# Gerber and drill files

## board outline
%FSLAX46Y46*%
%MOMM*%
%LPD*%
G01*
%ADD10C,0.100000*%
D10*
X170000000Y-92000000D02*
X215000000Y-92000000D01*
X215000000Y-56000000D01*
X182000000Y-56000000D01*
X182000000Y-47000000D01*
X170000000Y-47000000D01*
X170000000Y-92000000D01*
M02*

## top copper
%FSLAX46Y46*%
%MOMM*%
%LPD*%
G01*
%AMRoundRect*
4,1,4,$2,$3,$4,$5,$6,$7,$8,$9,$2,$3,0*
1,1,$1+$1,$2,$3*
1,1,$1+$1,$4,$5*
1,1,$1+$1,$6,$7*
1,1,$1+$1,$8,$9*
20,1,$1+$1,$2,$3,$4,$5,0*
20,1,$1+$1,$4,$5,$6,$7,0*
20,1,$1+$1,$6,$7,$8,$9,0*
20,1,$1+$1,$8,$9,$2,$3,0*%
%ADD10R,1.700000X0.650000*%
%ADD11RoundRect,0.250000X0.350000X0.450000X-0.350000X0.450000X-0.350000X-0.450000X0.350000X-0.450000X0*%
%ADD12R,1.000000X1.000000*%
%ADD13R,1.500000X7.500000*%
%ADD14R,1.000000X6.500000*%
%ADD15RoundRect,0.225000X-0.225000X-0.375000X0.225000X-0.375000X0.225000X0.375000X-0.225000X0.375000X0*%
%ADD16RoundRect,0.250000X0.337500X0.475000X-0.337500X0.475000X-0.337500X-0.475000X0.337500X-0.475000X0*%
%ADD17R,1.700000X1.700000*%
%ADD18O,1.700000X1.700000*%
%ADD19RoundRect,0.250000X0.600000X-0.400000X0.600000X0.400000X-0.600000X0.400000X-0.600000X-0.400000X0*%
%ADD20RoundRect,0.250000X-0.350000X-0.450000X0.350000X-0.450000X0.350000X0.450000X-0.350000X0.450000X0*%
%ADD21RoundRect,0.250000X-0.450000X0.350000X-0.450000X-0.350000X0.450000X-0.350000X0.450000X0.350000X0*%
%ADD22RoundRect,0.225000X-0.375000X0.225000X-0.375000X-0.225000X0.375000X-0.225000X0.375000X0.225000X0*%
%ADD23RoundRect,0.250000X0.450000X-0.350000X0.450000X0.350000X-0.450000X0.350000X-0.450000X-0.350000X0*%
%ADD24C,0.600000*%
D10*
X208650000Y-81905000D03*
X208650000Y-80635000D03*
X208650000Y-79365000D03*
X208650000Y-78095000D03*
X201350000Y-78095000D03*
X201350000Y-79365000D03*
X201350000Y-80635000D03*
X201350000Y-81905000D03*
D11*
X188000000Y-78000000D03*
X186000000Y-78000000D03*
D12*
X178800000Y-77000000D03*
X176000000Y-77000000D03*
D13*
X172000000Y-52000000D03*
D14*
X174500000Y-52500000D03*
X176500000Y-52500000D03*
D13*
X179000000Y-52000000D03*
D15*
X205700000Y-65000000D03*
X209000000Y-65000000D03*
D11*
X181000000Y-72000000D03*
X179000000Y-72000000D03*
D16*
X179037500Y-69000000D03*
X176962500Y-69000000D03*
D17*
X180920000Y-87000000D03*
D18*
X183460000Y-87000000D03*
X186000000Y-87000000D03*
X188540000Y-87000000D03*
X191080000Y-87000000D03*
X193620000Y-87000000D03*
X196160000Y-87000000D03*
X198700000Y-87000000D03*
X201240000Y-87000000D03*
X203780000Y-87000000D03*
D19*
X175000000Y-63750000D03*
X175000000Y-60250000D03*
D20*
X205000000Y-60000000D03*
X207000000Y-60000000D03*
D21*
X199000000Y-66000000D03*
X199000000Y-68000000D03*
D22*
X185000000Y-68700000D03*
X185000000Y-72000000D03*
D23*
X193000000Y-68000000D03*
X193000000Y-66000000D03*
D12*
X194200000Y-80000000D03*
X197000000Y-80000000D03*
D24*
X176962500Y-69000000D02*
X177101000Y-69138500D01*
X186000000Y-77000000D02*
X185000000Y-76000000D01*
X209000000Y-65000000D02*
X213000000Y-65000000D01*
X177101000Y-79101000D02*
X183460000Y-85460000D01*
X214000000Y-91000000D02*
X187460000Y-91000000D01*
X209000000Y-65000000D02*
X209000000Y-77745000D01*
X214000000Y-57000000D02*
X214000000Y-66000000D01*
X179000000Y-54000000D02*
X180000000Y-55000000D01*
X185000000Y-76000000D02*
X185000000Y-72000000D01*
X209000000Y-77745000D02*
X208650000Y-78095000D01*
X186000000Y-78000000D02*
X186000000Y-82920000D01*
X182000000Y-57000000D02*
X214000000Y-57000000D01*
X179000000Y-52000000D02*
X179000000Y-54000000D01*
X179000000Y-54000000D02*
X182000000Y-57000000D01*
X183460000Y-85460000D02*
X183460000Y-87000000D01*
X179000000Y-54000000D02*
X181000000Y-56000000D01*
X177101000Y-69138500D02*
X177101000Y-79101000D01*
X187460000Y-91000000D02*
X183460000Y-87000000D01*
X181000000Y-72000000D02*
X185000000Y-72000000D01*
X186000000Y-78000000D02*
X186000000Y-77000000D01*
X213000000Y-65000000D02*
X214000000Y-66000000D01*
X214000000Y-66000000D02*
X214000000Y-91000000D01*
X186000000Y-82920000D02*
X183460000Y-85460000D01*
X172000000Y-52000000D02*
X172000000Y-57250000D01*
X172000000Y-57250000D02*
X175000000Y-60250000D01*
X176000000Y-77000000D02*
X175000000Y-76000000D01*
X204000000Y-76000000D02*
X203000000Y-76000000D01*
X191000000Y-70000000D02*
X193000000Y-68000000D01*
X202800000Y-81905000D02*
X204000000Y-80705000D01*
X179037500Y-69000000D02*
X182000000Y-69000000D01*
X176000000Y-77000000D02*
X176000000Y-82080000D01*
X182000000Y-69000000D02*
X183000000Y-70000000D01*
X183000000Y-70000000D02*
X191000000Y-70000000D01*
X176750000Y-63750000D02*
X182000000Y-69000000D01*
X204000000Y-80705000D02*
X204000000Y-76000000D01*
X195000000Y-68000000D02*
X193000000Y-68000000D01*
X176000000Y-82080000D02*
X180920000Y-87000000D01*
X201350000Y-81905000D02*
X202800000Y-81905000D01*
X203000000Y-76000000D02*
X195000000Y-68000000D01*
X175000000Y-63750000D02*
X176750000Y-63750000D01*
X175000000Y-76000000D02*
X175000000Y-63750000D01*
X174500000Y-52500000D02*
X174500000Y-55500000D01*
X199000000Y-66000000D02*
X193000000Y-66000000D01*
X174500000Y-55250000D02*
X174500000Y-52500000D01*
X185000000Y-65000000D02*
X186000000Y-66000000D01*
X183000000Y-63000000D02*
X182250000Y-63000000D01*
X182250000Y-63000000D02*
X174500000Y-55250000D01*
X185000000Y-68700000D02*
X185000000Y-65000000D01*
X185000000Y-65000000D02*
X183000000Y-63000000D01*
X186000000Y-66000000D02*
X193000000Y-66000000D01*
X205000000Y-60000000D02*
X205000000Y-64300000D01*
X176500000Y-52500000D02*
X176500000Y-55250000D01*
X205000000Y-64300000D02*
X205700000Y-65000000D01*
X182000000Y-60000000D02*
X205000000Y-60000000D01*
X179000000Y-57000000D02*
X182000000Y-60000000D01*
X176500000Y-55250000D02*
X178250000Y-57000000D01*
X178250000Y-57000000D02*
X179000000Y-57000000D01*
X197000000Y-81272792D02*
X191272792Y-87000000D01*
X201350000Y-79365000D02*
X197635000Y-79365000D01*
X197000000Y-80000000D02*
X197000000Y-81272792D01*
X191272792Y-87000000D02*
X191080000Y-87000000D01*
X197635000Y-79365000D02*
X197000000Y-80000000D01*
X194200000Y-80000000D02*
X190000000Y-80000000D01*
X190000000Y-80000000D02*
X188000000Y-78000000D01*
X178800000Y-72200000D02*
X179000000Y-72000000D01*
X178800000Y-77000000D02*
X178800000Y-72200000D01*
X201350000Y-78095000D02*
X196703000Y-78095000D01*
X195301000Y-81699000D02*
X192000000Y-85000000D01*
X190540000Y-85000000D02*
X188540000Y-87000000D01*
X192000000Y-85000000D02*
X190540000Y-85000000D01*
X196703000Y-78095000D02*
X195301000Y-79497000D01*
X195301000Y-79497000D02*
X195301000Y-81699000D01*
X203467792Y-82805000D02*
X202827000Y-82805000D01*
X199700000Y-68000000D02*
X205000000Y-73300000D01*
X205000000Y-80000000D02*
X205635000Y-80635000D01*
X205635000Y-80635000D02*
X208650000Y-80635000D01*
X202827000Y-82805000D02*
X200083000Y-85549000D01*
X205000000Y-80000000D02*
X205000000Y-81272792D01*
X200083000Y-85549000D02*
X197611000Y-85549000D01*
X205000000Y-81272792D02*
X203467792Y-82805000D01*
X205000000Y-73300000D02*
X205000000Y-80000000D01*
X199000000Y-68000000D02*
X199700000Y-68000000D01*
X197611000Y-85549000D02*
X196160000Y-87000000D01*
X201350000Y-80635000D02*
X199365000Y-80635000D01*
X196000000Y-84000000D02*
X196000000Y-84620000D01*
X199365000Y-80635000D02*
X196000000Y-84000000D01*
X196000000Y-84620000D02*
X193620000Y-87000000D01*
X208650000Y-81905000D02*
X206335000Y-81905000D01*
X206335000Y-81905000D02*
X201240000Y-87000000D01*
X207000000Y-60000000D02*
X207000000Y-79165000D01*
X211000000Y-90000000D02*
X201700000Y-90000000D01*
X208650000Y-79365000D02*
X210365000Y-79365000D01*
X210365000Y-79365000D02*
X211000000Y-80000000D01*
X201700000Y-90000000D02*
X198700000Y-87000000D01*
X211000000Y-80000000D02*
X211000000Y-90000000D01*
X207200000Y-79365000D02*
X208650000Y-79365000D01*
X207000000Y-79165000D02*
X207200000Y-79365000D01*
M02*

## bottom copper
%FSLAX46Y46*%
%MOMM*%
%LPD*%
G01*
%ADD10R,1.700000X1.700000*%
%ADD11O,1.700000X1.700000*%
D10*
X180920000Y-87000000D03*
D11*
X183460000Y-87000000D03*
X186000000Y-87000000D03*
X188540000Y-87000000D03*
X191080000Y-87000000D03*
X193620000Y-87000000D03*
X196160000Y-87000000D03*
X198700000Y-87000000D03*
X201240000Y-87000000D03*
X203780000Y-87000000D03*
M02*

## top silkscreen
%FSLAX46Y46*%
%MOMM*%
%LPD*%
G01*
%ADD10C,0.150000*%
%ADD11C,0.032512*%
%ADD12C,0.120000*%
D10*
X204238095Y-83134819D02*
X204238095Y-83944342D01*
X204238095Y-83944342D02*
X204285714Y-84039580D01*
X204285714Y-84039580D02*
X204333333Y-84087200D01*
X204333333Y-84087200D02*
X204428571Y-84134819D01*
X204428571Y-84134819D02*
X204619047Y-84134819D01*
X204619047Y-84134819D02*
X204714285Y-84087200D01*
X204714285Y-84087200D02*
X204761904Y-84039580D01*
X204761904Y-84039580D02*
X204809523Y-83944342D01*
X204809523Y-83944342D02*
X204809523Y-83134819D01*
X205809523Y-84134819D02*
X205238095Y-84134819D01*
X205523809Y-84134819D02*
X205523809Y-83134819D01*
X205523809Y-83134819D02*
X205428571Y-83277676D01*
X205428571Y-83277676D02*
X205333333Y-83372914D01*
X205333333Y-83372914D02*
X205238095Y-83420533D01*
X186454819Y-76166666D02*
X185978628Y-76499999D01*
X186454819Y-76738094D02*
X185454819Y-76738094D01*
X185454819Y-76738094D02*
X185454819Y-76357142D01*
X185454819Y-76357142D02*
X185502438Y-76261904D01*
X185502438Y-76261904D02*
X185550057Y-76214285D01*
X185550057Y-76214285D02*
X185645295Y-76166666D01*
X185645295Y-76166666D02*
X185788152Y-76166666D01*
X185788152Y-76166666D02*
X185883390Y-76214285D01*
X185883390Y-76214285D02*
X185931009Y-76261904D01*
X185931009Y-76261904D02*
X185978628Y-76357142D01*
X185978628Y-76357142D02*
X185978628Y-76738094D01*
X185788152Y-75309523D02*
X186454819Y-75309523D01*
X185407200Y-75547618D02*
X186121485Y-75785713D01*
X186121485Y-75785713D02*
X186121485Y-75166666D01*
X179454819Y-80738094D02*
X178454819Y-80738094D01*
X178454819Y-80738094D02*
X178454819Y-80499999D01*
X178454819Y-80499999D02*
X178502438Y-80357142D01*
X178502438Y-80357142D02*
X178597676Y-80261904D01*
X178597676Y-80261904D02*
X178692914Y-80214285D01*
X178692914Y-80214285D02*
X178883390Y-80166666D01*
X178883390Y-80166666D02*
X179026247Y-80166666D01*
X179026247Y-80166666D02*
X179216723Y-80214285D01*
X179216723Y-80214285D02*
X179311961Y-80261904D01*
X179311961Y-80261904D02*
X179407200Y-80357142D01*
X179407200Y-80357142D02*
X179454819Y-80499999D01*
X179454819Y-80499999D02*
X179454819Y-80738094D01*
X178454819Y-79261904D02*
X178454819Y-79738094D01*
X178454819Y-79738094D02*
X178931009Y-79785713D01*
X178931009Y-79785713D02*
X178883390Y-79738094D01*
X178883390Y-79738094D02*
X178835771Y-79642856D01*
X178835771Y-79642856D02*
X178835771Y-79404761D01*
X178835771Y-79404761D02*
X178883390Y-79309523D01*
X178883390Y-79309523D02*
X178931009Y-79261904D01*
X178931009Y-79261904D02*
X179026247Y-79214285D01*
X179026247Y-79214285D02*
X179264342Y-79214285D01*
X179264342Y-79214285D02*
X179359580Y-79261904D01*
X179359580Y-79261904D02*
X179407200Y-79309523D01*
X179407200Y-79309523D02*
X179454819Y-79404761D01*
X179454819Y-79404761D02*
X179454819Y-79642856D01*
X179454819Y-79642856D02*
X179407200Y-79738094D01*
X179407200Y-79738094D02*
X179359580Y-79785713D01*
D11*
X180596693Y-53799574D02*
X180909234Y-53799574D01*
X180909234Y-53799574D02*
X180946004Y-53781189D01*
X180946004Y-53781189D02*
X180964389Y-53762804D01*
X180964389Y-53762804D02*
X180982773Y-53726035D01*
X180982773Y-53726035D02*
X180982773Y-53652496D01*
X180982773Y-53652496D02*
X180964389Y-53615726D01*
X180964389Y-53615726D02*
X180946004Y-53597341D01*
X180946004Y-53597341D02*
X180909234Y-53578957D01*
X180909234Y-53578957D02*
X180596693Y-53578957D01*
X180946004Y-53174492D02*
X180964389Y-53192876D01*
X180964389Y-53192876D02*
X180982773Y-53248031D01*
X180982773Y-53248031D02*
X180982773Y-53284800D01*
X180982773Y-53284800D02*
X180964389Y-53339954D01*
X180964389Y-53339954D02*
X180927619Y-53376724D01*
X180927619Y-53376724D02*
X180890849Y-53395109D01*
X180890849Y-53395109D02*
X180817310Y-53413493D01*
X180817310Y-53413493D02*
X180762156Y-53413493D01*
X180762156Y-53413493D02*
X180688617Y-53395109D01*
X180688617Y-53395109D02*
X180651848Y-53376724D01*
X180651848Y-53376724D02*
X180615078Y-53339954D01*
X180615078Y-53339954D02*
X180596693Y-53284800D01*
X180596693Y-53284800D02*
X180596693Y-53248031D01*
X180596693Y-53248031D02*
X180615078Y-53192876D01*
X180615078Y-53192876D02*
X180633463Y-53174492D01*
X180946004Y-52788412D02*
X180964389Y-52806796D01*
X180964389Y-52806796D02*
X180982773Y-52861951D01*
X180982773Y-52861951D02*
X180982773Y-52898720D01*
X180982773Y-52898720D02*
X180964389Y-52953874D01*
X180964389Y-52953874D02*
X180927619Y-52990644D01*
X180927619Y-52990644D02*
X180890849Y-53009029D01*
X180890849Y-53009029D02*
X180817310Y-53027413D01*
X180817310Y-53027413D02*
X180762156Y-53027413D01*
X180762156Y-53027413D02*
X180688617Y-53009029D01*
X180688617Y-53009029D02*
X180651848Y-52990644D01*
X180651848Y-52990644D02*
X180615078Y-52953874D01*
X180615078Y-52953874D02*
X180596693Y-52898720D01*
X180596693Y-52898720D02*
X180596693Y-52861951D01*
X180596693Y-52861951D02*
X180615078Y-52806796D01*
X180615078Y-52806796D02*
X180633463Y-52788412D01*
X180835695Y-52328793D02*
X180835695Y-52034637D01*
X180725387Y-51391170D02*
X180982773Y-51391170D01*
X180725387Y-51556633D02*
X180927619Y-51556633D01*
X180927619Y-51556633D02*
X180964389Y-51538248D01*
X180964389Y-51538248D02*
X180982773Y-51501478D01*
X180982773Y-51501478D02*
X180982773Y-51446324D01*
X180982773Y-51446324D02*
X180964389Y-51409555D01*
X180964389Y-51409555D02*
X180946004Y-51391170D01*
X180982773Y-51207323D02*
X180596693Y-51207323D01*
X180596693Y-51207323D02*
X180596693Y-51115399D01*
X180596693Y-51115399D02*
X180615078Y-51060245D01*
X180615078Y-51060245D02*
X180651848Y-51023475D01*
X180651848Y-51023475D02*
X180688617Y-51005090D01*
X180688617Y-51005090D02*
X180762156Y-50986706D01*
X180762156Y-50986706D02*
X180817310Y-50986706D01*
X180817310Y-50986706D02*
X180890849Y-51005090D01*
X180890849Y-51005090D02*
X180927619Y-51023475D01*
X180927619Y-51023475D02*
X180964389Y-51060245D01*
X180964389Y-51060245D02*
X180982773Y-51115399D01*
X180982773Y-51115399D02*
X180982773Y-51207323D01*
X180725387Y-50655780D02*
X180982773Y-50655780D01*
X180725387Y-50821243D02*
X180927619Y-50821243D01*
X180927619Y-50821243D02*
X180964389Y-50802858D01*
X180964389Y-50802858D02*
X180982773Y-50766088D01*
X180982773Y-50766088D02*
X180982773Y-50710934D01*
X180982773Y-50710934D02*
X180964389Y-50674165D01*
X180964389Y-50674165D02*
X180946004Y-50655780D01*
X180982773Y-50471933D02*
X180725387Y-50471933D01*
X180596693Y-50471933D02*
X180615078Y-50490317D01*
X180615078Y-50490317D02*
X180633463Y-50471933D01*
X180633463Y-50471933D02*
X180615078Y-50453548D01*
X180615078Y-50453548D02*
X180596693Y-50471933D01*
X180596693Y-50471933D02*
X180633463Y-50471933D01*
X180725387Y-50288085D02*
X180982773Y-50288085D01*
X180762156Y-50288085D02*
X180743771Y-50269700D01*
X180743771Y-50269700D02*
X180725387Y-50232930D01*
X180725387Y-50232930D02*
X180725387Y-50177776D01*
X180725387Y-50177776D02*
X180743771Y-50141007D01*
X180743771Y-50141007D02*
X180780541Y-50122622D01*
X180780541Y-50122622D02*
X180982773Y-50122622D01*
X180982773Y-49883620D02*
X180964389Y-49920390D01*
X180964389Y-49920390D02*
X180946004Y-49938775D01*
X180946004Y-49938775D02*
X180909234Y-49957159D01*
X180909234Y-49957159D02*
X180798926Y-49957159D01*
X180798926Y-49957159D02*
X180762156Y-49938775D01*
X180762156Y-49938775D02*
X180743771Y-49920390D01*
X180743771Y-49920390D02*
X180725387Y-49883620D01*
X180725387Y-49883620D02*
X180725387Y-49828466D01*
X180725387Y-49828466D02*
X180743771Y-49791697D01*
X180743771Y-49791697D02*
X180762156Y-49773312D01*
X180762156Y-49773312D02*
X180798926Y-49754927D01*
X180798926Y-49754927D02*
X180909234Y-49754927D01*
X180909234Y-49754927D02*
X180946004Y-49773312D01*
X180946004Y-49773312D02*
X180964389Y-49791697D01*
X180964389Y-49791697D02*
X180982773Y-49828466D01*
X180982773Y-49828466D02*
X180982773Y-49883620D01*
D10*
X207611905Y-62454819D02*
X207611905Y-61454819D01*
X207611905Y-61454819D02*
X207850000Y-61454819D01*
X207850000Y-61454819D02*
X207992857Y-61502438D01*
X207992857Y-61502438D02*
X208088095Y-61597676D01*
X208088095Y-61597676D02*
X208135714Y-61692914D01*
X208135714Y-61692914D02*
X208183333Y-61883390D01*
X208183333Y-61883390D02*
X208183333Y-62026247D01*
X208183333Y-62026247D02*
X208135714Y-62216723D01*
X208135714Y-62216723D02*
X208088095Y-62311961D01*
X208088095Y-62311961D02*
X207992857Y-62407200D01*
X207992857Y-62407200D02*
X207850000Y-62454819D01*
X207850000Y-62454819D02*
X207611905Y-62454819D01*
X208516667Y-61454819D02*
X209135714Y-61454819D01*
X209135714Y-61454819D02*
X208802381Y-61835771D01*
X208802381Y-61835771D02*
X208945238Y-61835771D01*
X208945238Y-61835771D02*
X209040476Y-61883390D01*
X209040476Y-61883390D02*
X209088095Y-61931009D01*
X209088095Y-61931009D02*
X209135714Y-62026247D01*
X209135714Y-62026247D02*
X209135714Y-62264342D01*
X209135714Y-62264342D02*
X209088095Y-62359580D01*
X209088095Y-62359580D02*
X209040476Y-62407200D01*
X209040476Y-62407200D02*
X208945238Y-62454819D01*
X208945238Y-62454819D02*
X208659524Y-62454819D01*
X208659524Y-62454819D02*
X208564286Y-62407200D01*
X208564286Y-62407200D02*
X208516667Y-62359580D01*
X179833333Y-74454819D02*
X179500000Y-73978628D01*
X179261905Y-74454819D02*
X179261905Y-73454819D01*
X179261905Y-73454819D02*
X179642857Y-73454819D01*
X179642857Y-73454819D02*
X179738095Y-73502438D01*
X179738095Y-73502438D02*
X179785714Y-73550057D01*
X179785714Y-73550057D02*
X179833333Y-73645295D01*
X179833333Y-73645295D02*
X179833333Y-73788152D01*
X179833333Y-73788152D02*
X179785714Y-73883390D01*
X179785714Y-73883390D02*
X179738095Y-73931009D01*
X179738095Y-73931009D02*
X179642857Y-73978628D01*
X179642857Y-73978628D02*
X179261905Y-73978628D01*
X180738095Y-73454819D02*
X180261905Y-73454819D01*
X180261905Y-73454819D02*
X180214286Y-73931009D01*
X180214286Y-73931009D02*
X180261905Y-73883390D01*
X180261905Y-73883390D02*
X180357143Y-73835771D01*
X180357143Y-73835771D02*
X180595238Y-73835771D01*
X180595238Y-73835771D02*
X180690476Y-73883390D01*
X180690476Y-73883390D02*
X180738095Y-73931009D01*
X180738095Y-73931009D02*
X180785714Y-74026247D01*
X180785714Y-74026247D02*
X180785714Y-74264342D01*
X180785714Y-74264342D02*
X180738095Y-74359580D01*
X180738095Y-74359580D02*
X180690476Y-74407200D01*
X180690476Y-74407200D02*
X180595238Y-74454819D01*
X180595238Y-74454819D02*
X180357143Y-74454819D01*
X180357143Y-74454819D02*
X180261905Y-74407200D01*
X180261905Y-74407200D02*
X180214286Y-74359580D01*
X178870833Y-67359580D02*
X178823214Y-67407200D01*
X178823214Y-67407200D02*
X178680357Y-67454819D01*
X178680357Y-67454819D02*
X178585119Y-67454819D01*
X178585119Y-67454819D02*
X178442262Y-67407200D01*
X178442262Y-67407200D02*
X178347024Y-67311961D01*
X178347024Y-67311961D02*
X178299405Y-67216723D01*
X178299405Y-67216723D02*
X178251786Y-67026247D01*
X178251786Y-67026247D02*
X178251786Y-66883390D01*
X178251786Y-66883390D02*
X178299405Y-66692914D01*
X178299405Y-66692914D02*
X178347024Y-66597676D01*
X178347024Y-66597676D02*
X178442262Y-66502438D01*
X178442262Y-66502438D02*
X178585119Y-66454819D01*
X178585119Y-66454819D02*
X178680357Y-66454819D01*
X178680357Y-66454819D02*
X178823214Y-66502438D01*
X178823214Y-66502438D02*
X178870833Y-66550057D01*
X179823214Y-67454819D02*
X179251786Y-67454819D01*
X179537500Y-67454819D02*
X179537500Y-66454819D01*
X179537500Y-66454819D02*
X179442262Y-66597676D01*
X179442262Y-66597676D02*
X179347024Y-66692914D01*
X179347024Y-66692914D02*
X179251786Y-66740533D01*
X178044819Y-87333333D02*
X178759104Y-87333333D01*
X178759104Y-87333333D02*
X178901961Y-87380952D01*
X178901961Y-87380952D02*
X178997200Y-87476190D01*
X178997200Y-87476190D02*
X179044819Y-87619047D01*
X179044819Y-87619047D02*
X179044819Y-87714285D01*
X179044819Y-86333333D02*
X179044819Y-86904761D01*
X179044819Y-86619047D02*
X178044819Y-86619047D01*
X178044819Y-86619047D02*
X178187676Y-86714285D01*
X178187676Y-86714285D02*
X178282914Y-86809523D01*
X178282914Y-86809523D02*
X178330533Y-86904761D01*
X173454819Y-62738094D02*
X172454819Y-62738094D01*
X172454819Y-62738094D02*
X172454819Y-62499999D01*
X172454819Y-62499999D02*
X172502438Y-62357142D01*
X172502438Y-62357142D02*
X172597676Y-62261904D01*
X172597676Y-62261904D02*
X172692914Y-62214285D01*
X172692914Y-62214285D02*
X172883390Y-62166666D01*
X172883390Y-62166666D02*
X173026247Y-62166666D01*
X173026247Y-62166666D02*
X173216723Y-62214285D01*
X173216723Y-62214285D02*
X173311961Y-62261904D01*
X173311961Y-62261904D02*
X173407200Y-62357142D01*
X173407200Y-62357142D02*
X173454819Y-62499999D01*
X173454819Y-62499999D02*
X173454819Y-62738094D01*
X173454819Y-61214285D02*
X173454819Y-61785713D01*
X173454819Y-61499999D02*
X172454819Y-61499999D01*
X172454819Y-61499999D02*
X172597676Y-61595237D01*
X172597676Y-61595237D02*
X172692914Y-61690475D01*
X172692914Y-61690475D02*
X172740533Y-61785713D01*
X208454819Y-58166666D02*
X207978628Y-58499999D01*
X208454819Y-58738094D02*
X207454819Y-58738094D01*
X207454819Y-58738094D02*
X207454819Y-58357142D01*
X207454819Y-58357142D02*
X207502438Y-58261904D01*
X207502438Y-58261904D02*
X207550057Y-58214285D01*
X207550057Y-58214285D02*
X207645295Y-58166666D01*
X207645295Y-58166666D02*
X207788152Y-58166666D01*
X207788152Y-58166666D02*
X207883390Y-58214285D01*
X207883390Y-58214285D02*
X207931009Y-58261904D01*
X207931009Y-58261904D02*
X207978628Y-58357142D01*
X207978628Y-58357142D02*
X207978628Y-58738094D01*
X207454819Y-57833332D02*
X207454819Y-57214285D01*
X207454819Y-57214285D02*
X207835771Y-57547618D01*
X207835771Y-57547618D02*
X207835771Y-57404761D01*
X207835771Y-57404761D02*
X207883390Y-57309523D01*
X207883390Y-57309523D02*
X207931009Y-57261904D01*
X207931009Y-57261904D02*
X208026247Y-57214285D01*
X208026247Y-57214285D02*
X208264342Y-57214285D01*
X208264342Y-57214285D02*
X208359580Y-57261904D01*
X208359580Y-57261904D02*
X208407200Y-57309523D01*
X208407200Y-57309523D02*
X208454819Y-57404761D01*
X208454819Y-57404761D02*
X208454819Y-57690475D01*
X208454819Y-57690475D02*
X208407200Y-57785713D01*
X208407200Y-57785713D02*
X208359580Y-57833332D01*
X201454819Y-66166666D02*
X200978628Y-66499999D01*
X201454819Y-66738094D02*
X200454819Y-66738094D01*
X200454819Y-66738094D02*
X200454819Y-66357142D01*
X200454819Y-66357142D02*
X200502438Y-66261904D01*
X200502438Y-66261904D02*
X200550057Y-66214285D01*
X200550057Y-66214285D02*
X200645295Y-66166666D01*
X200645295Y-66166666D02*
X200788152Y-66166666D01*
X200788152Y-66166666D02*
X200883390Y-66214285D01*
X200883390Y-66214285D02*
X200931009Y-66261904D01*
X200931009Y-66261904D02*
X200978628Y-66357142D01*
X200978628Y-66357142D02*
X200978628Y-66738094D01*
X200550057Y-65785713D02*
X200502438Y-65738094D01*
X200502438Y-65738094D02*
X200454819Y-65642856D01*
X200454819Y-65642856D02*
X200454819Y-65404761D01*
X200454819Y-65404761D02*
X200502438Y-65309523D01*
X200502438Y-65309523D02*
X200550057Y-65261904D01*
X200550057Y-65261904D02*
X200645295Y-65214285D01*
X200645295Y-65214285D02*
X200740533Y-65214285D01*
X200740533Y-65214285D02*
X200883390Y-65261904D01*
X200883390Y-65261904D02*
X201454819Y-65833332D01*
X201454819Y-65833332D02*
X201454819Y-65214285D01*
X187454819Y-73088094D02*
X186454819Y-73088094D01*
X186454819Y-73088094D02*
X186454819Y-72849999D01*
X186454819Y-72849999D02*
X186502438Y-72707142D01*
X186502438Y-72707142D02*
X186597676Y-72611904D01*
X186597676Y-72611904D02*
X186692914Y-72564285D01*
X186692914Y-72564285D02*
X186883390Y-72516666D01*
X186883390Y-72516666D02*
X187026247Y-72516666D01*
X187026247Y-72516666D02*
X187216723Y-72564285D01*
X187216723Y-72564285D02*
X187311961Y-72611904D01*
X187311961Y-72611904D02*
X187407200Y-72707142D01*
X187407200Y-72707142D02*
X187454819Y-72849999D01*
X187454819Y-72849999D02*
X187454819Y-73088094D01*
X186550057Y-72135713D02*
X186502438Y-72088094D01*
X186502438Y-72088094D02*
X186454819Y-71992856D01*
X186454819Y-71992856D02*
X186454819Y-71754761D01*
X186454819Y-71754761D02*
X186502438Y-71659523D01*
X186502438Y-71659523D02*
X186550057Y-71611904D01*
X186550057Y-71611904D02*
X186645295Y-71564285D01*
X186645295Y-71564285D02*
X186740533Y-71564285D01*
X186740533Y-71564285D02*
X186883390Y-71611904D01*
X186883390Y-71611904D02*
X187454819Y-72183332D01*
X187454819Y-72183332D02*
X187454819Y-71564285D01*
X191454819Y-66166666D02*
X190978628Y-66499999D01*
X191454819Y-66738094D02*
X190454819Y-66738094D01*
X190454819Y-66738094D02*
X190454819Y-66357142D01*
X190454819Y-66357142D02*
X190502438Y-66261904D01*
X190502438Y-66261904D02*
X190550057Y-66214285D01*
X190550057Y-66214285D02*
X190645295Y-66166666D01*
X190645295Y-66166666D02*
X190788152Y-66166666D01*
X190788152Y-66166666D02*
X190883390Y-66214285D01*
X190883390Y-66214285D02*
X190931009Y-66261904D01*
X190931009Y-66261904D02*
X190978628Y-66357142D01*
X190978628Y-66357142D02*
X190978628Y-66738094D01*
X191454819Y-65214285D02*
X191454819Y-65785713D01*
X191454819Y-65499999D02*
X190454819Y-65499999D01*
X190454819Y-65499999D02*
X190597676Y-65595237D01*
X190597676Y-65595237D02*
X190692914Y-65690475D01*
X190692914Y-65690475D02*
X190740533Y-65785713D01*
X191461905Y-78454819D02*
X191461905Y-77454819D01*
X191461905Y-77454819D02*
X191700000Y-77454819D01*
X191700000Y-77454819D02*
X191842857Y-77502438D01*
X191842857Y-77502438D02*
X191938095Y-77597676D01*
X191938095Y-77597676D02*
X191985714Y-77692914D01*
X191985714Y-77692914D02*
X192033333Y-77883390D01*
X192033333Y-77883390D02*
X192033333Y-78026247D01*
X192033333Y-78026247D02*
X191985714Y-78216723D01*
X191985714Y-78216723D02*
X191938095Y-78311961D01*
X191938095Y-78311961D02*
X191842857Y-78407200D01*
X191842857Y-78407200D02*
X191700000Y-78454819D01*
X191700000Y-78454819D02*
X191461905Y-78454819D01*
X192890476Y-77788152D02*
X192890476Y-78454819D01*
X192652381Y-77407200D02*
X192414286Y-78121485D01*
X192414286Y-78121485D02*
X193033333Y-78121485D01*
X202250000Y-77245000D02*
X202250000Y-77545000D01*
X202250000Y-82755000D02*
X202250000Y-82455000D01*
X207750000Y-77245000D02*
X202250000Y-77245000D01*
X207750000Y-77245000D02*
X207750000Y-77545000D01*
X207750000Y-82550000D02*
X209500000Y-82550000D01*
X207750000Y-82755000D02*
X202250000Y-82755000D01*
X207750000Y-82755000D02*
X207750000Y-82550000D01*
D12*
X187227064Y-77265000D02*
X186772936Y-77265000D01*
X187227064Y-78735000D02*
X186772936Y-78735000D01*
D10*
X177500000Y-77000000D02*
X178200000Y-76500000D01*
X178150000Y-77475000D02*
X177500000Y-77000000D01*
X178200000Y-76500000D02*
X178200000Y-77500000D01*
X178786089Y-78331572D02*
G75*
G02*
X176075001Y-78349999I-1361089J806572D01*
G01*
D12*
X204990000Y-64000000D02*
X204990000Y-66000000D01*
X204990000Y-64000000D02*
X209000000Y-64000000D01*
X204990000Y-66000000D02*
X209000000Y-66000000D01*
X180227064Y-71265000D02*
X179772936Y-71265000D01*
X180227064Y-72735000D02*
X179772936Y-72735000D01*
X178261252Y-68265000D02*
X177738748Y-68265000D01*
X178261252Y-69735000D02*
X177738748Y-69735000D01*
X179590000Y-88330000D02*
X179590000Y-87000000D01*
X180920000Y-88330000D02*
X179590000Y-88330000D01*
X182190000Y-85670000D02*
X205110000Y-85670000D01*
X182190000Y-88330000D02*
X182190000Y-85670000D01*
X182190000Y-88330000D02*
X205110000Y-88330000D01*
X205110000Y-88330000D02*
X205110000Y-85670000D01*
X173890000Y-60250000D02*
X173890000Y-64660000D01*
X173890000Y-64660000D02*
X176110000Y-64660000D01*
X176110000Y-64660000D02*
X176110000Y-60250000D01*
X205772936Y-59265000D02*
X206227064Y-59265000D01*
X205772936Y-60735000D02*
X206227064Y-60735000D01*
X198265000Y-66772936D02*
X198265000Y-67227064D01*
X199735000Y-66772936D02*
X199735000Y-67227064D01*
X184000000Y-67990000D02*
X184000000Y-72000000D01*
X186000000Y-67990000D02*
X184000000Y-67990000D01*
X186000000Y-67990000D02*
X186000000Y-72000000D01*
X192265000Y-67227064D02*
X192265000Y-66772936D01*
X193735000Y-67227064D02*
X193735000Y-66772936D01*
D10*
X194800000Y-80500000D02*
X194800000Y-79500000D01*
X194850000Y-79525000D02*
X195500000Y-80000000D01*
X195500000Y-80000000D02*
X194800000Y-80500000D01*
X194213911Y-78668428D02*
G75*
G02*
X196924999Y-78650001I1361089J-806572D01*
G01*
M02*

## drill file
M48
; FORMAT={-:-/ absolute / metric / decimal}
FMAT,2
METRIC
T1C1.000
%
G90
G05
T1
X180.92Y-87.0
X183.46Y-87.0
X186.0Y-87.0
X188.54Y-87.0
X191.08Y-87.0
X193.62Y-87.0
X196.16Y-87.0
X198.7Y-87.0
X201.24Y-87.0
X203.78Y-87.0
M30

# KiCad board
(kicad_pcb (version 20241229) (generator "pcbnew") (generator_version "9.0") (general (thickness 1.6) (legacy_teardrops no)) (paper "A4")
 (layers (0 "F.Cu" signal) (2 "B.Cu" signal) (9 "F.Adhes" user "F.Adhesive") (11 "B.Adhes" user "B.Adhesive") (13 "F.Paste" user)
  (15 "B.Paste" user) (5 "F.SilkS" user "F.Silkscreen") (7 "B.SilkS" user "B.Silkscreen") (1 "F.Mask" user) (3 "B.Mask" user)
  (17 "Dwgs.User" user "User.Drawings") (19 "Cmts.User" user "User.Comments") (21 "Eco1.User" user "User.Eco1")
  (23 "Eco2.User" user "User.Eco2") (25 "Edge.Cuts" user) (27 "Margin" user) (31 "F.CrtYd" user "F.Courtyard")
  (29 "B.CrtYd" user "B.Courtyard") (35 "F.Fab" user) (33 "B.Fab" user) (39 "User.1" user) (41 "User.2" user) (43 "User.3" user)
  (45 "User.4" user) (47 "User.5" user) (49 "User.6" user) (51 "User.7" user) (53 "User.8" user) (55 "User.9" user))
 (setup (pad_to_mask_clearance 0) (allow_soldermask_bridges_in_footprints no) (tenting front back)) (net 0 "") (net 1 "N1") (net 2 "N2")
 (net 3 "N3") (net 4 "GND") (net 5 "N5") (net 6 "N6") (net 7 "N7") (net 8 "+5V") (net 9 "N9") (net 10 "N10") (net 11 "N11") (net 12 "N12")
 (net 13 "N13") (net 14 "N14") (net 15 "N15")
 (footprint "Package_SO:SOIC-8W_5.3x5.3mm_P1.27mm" (layer "F.Cu") (at 205 80 180)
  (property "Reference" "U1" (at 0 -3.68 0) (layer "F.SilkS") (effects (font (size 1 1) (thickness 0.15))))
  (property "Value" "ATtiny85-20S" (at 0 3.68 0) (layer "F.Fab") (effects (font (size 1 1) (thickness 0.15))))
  (fp_line (start 2.75 2.755) (end 2.75 2.455) (stroke (width 0.15) (type solid)) (layer "F.SilkS"))
  (fp_line (start 2.75 -2.755) (end 2.75 -2.455) (stroke (width 0.15) (type solid)) (layer "F.SilkS"))
  (fp_line (start -2.75 2.755) (end 2.75 2.755) (stroke (width 0.15) (type solid)) (layer "F.SilkS"))
  (fp_line (start -2.75 2.755) (end -2.75 2.455) (stroke (width 0.15) (type solid)) (layer "F.SilkS"))
  (fp_line (start -2.75 -2.55) (end -4.5 -2.55) (stroke (width 0.15) (type solid)) (layer "F.SilkS"))
  (fp_line (start -2.75 -2.755) (end 2.75 -2.755) (stroke (width 0.15) (type solid)) (layer "F.SilkS"))
  (fp_line (start -2.75 -2.755) (end -2.75 -2.55) (stroke (width 0.15) (type solid)) (layer "F.SilkS"))
  (pad "1" smd rect (at -3.65 -1.905 180) (size 1.7 0.65) (layers "F.Cu" "F.Mask" "F.Paste") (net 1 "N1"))
  (pad "2" smd rect (at -3.65 -0.635 180) (size 1.7 0.65) (layers "F.Cu" "F.Mask" "F.Paste") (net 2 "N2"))
  (pad "3" smd rect (at -3.65 0.635 180) (size 1.7 0.65) (layers "F.Cu" "F.Mask" "F.Paste") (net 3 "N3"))
  (pad "4" smd rect (at -3.65 1.905 180) (size 1.7 0.65) (layers "F.Cu" "F.Mask" "F.Paste") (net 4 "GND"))
  (pad "5" smd rect (at 3.65 1.905 180) (size 1.7 0.65) (layers "F.Cu" "F.Mask" "F.Paste") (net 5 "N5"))
  (pad "6" smd rect (at 3.65 0.635 180) (size 1.7 0.65) (layers "F.Cu" "F.Mask" "F.Paste") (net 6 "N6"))
  (pad "7" smd rect (at 3.65 -0.635 180) (size 1.7 0.65) (layers "F.Cu" "F.Mask" "F.Paste") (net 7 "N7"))
  (pad "8" smd rect (at 3.65 -1.905 180) (size 1.7 0.65) (layers "F.Cu" "F.Mask" "F.Paste") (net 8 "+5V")))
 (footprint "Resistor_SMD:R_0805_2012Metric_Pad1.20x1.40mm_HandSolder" (layer "F.Cu") (at 187 78 180)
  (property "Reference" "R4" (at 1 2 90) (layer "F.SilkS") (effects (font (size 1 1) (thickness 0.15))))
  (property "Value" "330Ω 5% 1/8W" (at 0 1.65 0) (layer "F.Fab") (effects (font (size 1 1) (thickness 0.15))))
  (fp_line (start -0.227064 0.735) (end 0.227064 0.735) (stroke (width 0.12) (type solid)) (layer "F.SilkS"))
  (fp_line (start -0.227064 -0.735) (end 0.227064 -0.735) (stroke (width 0.12) (type solid)) (layer "F.SilkS"))
  (pad "1" smd roundrect (at -1 0 180) (size 1.2 1.4) (layers "F.Cu" "F.Mask" "F.Paste") (roundrect_rratio 0.208333) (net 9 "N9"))
  (pad "2" smd roundrect (at 1 0 180) (size 1.2 1.4) (layers "F.Cu" "F.Mask" "F.Paste") (roundrect_rratio 0.208333) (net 4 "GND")))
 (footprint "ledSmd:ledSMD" (layer "F.Cu") (at 177 77 180)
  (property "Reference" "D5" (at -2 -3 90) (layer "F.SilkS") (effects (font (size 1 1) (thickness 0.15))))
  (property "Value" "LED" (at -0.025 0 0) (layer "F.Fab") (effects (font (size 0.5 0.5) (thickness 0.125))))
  (fp_line (start -0.5 0) (end -1.2 0.5) (stroke (width 0.15) (type solid)) (layer "F.SilkS"))
  (fp_line (start -1.15 -0.475) (end -0.5 0) (stroke (width 0.15) (type solid)) (layer "F.SilkS"))
  (fp_line (start -1.2 0.5) (end -1.2 -0.5) (stroke (width 0.15) (type solid)) (layer "F.SilkS"))
  (fp_arc (start -1.786089 -1.331572) (mid -0.435753 -2.107089) (end 0.924999 -1.349999) (stroke (width 0.15) (type solid))
   (layer "F.SilkS"))
  (pad "1" smd rect (at -1.8 0 180) (size 1 1) (layers "F.Cu" "F.Mask" "F.Paste") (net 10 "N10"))
  (pad "2" smd rect (at 1 0 180) (size 1 1) (layers "F.Cu" "F.Mask" "F.Paste") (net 8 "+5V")))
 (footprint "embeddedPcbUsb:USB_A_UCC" (layer "F.Cu") (at 175.5 52.2 -90)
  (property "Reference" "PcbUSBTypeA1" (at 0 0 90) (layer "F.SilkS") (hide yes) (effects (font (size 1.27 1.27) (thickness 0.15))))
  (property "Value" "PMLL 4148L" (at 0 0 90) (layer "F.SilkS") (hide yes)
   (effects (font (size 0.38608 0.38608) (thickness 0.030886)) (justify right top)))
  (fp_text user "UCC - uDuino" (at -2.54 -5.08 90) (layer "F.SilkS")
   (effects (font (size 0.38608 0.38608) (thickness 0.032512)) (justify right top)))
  (pad "1" smd rect (at -0.2 3.5 270) (size 7.5 1.5) (layers "F.Cu" "F.Mask" "F.Paste") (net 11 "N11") (solder_mask_margin 0.1016))
  (pad "2" smd rect (at 0.3 1 270) (size 6.5 1) (layers "F.Cu" "F.Mask" "F.Paste") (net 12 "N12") (solder_mask_margin 0.1016))
  (pad "3" smd rect (at 0.3 -1 270) (size 6.5 1) (layers "F.Cu" "F.Mask" "F.Paste") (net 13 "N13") (solder_mask_margin 0.1016))
  (pad "4" smd rect (at -0.2 -3.5 270) (size 7.5 1.5) (layers "F.Cu" "F.Mask" "F.Paste") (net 4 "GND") (solder_mask_margin 0.1016)))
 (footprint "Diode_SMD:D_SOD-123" (layer "F.Cu") (at 207.35 65)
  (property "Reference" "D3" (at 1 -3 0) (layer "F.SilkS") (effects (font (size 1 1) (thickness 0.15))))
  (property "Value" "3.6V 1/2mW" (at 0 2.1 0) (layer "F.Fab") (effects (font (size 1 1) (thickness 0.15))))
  (fp_line (start -2.36 -1) (end -2.36 1) (stroke (width 0.12) (type solid)) (layer "F.SilkS"))
  (fp_line (start -2.36 -1) (end 1.65 -1) (stroke (width 0.12) (type solid)) (layer "F.SilkS"))
  (fp_line (start -2.36 1) (end 1.65 1) (stroke (width 0.12) (type solid)) (layer "F.SilkS"))
  (pad "1" smd roundrect (at -1.65 0) (size 0.9 1.2) (layers "F.Cu" "F.Mask" "F.Paste") (roundrect_rratio 0.25) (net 13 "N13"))
  (pad "2" smd roundrect (at 1.65 0) (size 0.9 1.2) (layers "F.Cu" "F.Mask" "F.Paste") (roundrect_rratio 0.25) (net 4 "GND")))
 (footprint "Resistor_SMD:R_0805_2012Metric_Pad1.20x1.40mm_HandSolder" (layer "F.Cu") (at 180 72 180)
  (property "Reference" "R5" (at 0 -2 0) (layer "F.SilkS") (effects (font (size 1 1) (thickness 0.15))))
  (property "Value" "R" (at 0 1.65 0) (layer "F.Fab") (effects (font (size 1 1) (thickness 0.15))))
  (fp_line (start -0.227064 0.735) (end 0.227064 0.735) (stroke (width 0.12) (type solid)) (layer "F.SilkS"))
  (fp_line (start -0.227064 -0.735) (end 0.227064 -0.735) (stroke (width 0.12) (type solid)) (layer "F.SilkS"))
  (pad "1" smd roundrect (at -1 0 180) (size 1.2 1.4) (layers "F.Cu" "F.Mask" "F.Paste") (roundrect_rratio 0.208333) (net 4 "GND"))
  (pad "2" smd roundrect (at 1 0 180) (size 1.2 1.4) (layers "F.Cu" "F.Mask" "F.Paste") (roundrect_rratio 0.208333) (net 10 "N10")))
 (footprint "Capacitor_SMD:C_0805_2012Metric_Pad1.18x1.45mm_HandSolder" (layer "F.Cu") (at 178 69 180)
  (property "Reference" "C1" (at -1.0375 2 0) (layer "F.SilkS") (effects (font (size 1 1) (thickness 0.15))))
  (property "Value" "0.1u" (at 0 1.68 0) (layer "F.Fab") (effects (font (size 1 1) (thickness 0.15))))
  (fp_line (start -0.261252 0.735) (end 0.261252 0.735) (stroke (width 0.12) (type solid)) (layer "F.SilkS"))
  (fp_line (start -0.261252 -0.735) (end 0.261252 -0.735) (stroke (width 0.12) (type solid)) (layer "F.SilkS"))
  (pad "1" smd roundrect (at -1.0375 0 180) (size 1.175 1.45) (layers "F.Cu" "F.Mask" "F.Paste") (roundrect_rratio 0.212766) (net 8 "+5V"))
  (pad "2" smd roundrect (at 1.0375 0 180) (size 1.175 1.45) (layers "F.Cu" "F.Mask" "F.Paste") (roundrect_rratio 0.212766) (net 4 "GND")))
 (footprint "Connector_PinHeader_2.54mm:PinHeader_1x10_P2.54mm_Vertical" (layer "F.Cu") (at 180.92 87 90)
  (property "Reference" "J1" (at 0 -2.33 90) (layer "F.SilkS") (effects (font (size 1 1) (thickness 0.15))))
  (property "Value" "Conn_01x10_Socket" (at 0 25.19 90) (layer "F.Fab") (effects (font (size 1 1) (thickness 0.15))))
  (fp_line (start -1.33 -1.33) (end 0 -1.33) (stroke (width 0.12) (type solid)) (layer "F.SilkS"))
  (fp_line (start -1.33 0) (end -1.33 -1.33) (stroke (width 0.12) (type solid)) (layer "F.SilkS"))
  (fp_line (start 1.33 1.27) (end 1.33 24.19) (stroke (width 0.12) (type solid)) (layer "F.SilkS"))
  (fp_line (start -1.33 1.27) (end 1.33 1.27) (stroke (width 0.12) (type solid)) (layer "F.SilkS"))
  (fp_line (start -1.33 1.27) (end -1.33 24.19) (stroke (width 0.12) (type solid)) (layer "F.SilkS"))
  (fp_line (start -1.33 24.19) (end 1.33 24.19) (stroke (width 0.12) (type solid)) (layer "F.SilkS"))
  (pad "1" thru_hole rect (at 0 0 90) (size 1.7 1.7) (drill 1) (layers "*.Cu" "*.Mask") (remove_unused_layers no) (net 8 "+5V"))
  (pad "2" thru_hole oval (at 0 2.54 90) (size 1.7 1.7) (drill 1) (layers "*.Cu" "*.Mask") (remove_unused_layers no) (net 4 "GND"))
  (pad "3" thru_hole oval (at 0 5.08 90) (size 1.7 1.7) (drill 1) (layers "*.Cu" "*.Mask") (remove_unused_layers no) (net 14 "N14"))
  (pad "4" thru_hole oval (at 0 7.62 90) (size 1.7 1.7) (drill 1) (layers "*.Cu" "*.Mask") (remove_unused_layers no) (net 5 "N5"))
  (pad "5" thru_hole oval (at 0 10.16 90) (size 1.7 1.7) (drill 1) (layers "*.Cu" "*.Mask") (remove_unused_layers no) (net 6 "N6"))
  (pad "6" thru_hole oval (at 0 12.7 90) (size 1.7 1.7) (drill 1) (layers "*.Cu" "*.Mask") (remove_unused_layers no) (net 7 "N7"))
  (pad "7" thru_hole oval (at 0 15.24 90) (size 1.7 1.7) (drill 1) (layers "*.Cu" "*.Mask") (remove_unused_layers no) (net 2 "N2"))
  (pad "8" thru_hole oval (at 0 17.78 90) (size 1.7 1.7) (drill 1) (layers "*.Cu" "*.Mask") (remove_unused_layers no) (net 3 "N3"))
  (pad "9" thru_hole oval (at 0 20.32 90) (size 1.7 1.7) (drill 1) (layers "*.Cu" "*.Mask") (remove_unused_layers no) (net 1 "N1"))
  (pad "10" thru_hole oval (at 0 22.86 90) (size 1.7 1.7) (drill 1) (layers "*.Cu" "*.Mask") (remove_unused_layers no) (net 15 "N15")))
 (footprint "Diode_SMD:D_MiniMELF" (layer "F.Cu") (at 175 62 90)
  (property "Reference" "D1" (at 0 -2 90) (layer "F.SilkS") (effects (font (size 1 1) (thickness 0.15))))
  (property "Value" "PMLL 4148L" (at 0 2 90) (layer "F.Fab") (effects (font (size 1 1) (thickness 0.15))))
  (fp_line (start 1.75 -1.11) (end -2.66 -1.11) (stroke (width 0.12) (type solid)) (layer "F.SilkS"))
  (fp_line (start -2.66 -1.11) (end -2.66 1.11) (stroke (width 0.12) (type solid)) (layer "F.SilkS"))
  (fp_line (start -2.66 1.11) (end 1.75 1.11) (stroke (width 0.12) (type solid)) (layer "F.SilkS"))
  (pad "1" smd roundrect (at -1.75 0 90) (size 1.3 1.7) (layers "F.Cu" "F.Mask" "F.Paste") (roundrect_rratio 0.1923076923) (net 8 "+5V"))
  (pad "2" smd roundrect (at 1.75 0 90) (size 1.3 1.7) (layers "F.Cu" "F.Mask" "F.Paste") (roundrect_rratio 0.1923076923) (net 11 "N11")))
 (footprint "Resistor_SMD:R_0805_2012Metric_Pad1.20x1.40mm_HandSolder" (layer "F.Cu") (at 206 60)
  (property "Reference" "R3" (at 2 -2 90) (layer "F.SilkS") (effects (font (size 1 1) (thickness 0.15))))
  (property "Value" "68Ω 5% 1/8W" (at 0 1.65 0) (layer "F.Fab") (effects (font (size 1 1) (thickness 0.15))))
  (fp_line (start -0.227064 -0.735) (end 0.227064 -0.735) (stroke (width 0.12) (type solid)) (layer "F.SilkS"))
  (fp_line (start -0.227064 0.735) (end 0.227064 0.735) (stroke (width 0.12) (type solid)) (layer "F.SilkS"))
  (pad "1" smd roundrect (at -1 0) (size 1.2 1.4) (layers "F.Cu" "F.Mask" "F.Paste") (roundrect_rratio 0.208333) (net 13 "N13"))
  (pad "2" smd roundrect (at 1 0) (size 1.2 1.4) (layers "F.Cu" "F.Mask" "F.Paste") (roundrect_rratio 0.208333) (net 3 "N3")))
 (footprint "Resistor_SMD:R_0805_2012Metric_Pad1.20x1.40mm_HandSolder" (layer "F.Cu") (at 199 67 -90)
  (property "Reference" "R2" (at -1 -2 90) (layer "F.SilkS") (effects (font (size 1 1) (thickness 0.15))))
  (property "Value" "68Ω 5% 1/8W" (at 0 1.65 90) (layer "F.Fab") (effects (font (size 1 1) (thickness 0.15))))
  (fp_line (start -0.227064 0.735) (end 0.227064 0.735) (stroke (width 0.12) (type solid)) (layer "F.SilkS"))
  (fp_line (start -0.227064 -0.735) (end 0.227064 -0.735) (stroke (width 0.12) (type solid)) (layer "F.SilkS"))
  (pad "1" smd roundrect (at -1 0 270) (size 1.2 1.4) (layers "F.Cu" "F.Mask" "F.Paste") (roundrect_rratio 0.208333) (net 12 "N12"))
  (pad "2" smd roundrect (at 1 0 270) (size 1.2 1.4) (layers "F.Cu" "F.Mask" "F.Paste") (roundrect_rratio 0.208333) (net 2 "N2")))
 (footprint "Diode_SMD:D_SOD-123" (layer "F.Cu") (at 185 70.35 -90)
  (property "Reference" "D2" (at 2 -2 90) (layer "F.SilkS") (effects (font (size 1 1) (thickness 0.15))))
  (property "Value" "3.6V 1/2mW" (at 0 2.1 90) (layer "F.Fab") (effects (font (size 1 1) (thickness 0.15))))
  (fp_line (start -2.36 1) (end 1.65 1) (stroke (width 0.12) (type solid)) (layer "F.SilkS"))
  (fp_line (start -2.36 -1) (end -2.36 1) (stroke (width 0.12) (type solid)) (layer "F.SilkS"))
  (fp_line (start -2.36 -1) (end 1.65 -1) (stroke (width 0.12) (type solid)) (layer "F.SilkS"))
  (pad "1" smd roundrect (at -1.65 0 270) (size 0.9 1.2) (layers "F.Cu" "F.Mask" "F.Paste") (roundrect_rratio 0.25) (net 12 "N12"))
  (pad "2" smd roundrect (at 1.65 0 270) (size 0.9 1.2) (layers "F.Cu" "F.Mask" "F.Paste") (roundrect_rratio 0.25) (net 4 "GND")))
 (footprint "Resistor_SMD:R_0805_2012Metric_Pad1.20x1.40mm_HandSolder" (layer "F.Cu") (at 193 67 90)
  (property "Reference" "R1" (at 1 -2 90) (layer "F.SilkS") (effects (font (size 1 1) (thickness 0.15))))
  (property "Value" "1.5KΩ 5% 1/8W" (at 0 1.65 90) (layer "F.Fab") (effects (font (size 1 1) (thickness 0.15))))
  (fp_line (start -0.227064 -0.735) (end 0.227064 -0.735) (stroke (width 0.12) (type solid)) (layer "F.SilkS"))
  (fp_line (start -0.227064 0.735) (end 0.227064 0.735) (stroke (width 0.12) (type solid)) (layer "F.SilkS"))
  (pad "1" smd roundrect (at -1 0 90) (size 1.2 1.4) (layers "F.Cu" "F.Mask" "F.Paste") (roundrect_rratio 0.208333) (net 8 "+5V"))
  (pad "2" smd roundrect (at 1 0 90) (size 1.2 1.4) (layers "F.Cu" "F.Mask" "F.Paste") (roundrect_rratio 0.208333) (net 12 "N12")))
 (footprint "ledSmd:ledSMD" (layer "F.Cu") (at 196 80)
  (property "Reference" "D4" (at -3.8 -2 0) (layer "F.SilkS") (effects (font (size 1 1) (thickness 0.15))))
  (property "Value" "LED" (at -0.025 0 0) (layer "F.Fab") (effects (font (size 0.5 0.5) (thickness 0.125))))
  (fp_line (start -1.2 0.5) (end -1.2 -0.5) (stroke (width 0.15) (type solid)) (layer "F.SilkS"))
  (fp_line (start -1.15 -0.475) (end -0.5 0) (stroke (width 0.15) (type solid)) (layer "F.SilkS"))
  (fp_line (start -0.5 0) (end -1.2 0.5) (stroke (width 0.15) (type solid)) (layer "F.SilkS"))
  (fp_arc (start -1.786089 -1.331572) (mid -0.435753 -2.107089) (end 0.924999 -1.349999) (stroke (width 0.15) (type solid))
   (layer "F.SilkS"))
  (pad "1" smd rect (at -1.8 0) (size 1 1) (layers "F.Cu" "F.Mask" "F.Paste") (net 9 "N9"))
  (pad "2" smd rect (at 1 0) (size 1 1) (layers "F.Cu" "F.Mask" "F.Paste") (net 6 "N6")))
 (gr_poly
  (pts (xy 170 92) (xy 215 92) (xy 215 56) (xy 182 56) (xy 182 47) (xy 170 47)) (stroke (width 0.1) (type solid)) (fill no)
  (layer "Edge.Cuts"))
 (segment (start 176.9625 69) (end 177.101 69.1385) (width 0.6) (layer "F.Cu") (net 4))
 (segment (start 186 77) (end 185 76) (width 0.6) (layer "F.Cu") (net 4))
 (segment (start 209 65) (end 213 65) (width 0.6) (layer "F.Cu") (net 4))
 (segment (start 177.101 79.101) (end 183.46 85.46) (width 0.6) (layer "F.Cu") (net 4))
 (segment (start 214 91) (end 187.46 91) (width 0.6) (layer "F.Cu") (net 4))
 (segment (start 209 65) (end 209 77.745) (width 0.6) (layer "F.Cu") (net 4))
 (segment (start 214 57) (end 214 66) (width 0.6) (layer "F.Cu") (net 4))
 (segment (start 179 54) (end 180 55) (width 0.6) (layer "F.Cu") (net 4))
 (segment (start 185 76) (end 185 72) (width 0.6) (layer "F.Cu") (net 4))
 (segment (start 209 77.745) (end 208.65 78.095) (width 0.6) (layer "F.Cu") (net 4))
 (segment (start 186 78) (end 186 82.92) (width 0.6) (layer "F.Cu") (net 4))
 (segment (start 182 57) (end 214 57) (width 0.6) (layer "F.Cu") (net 4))
 (segment (start 179 52) (end 179 54) (width 0.6) (layer "F.Cu") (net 4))
 (segment (start 179 54) (end 182 57) (width 0.6) (layer "F.Cu") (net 4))
 (segment (start 183.46 85.46) (end 183.46 87) (width 0.6) (layer "F.Cu") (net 4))
 (segment (start 179 54) (end 181 56) (width 0.6) (layer "F.Cu") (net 4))
 (segment (start 177.101 69.1385) (end 177.101 79.101) (width 0.6) (layer "F.Cu") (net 4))
 (segment (start 187.46 91) (end 183.46 87) (width 0.6) (layer "F.Cu") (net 4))
 (segment (start 181 72) (end 185 72) (width 0.6) (layer "F.Cu") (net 4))
 (segment (start 186 78) (end 186 77) (width 0.6) (layer "F.Cu") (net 4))
 (segment (start 213 65) (end 214 66) (width 0.6) (layer "F.Cu") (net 4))
 (segment (start 214 66) (end 214 91) (width 0.6) (layer "F.Cu") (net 4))
 (segment (start 186 82.92) (end 183.46 85.46) (width 0.6) (layer "F.Cu") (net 4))
 (segment (start 172 52) (end 172 57.25) (width 0.6) (layer "F.Cu") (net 11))
 (segment (start 172 57.25) (end 175 60.25) (width 0.6) (layer "F.Cu") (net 11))
 (segment (start 176 77) (end 175 76) (width 0.6) (layer "F.Cu") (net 8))
 (segment (start 204 76) (end 203 76) (width 0.6) (layer "F.Cu") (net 8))
 (segment (start 191 70) (end 193 68) (width 0.6) (layer "F.Cu") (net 8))
 (segment (start 202.8 81.905) (end 204 80.705) (width 0.6) (layer "F.Cu") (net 8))
 (segment (start 179.0375 69) (end 182 69) (width 0.6) (layer "F.Cu") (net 8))
 (segment (start 176 77) (end 176 82.08) (width 0.6) (layer "F.Cu") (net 8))
 (segment (start 182 69) (end 183 70) (width 0.6) (layer "F.Cu") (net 8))
 (segment (start 183 70) (end 191 70) (width 0.6) (layer "F.Cu") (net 8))
 (segment (start 176.75 63.75) (end 182 69) (width 0.6) (layer "F.Cu") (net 8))
 (segment (start 204 80.705) (end 204 76) (width 0.6) (layer "F.Cu") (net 8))
 (segment (start 195 68) (end 193 68) (width 0.6) (layer "F.Cu") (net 8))
 (segment (start 176 82.08) (end 180.92 87) (width 0.6) (layer "F.Cu") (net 8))
 (segment (start 201.35 81.905) (end 202.8 81.905) (width 0.6) (layer "F.Cu") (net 8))
 (segment (start 203 76) (end 195 68) (width 0.6) (layer "F.Cu") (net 8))
 (segment (start 175 63.75) (end 176.75 63.75) (width 0.6) (layer "F.Cu") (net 8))
 (segment (start 175 76) (end 175 63.75) (width 0.6) (layer "F.Cu") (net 8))
 (segment (start 174.5 52.5) (end 174.5 55.5) (width 0.6) (layer "F.Cu") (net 12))
 (segment (start 199 66) (end 193 66) (width 0.6) (layer "F.Cu") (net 12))
 (segment (start 174.5 55.25) (end 174.5 52.5) (width 0.6) (layer "F.Cu") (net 12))
 (segment (start 185 65) (end 186 66) (width 0.6) (layer "F.Cu") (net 12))
 (segment (start 183 63) (end 182.25 63) (width 0.6) (layer "F.Cu") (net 12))
 (segment (start 182.25 63) (end 174.5 55.25) (width 0.6) (layer "F.Cu") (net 12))
 (segment (start 185 68.7) (end 185 65) (width 0.6) (layer "F.Cu") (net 12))
 (segment (start 185 65) (end 183 63) (width 0.6) (layer "F.Cu") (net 12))
 (segment (start 186 66) (end 193 66) (width 0.6) (layer "F.Cu") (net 12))
 (segment (start 205 60) (end 205 64.3) (width 0.6) (layer "F.Cu") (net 13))
 (segment (start 176.5 52.5) (end 176.5 55.25) (width 0.6) (layer "F.Cu") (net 13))
 (segment (start 205 64.3) (end 205.7 65) (width 0.6) (layer "F.Cu") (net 13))
 (segment (start 182 60) (end 205 60) (width 0.6) (layer "F.Cu") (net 13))
 (segment (start 179 57) (end 182 60) (width 0.6) (layer "F.Cu") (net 13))
 (segment (start 176.5 55.25) (end 178.25 57) (width 0.6) (layer "F.Cu") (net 13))
 (segment (start 178.25 57) (end 179 57) (width 0.6) (layer "F.Cu") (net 13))
 (segment (start 197 81.272792) (end 191.272792 87) (width 0.6) (layer "F.Cu") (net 6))
 (segment (start 201.35 79.365) (end 197.635 79.365) (width 0.6) (layer "F.Cu") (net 6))
 (segment (start 197 80) (end 197 81.272792) (width 0.6) (layer "F.Cu") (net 6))
 (segment (start 191.272792 87) (end 191.08 87) (width 0.6) (layer "F.Cu") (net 6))
 (segment (start 197.635 79.365) (end 197 80) (width 0.6) (layer "F.Cu") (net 6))
 (segment (start 194.2 80) (end 190 80) (width 0.6) (layer "F.Cu") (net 9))
 (segment (start 190 80) (end 188 78) (width 0.6) (layer "F.Cu") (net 9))
 (segment (start 178.8 72.2) (end 179 72) (width 0.6) (layer "F.Cu") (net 10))
 (segment (start 178.8 77) (end 178.8 72.2) (width 0.6) (layer "F.Cu") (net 10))
 (segment (start 201.35 78.095) (end 196.703 78.095) (width 0.6) (layer "F.Cu") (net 5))
 (segment (start 195.301 81.699) (end 192 85) (width 0.6) (layer "F.Cu") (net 5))
 (segment (start 190.54 85) (end 188.54 87) (width 0.6) (layer "F.Cu") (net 5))
 (segment (start 192 85) (end 190.54 85) (width 0.6) (layer "F.Cu") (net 5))
 (segment (start 196.703 78.095) (end 195.301 79.497) (width 0.6) (layer "F.Cu") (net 5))
 (segment (start 195.301 79.497) (end 195.301 81.699) (width 0.6) (layer "F.Cu") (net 5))
 (segment (start 203.467792 82.805) (end 202.827 82.805) (width 0.6) (layer "F.Cu") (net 2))
 (segment (start 199.7 68) (end 205 73.3) (width 0.6) (layer "F.Cu") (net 2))
 (segment (start 205 80) (end 205.635 80.635) (width 0.6) (layer "F.Cu") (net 2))
 (segment (start 205.635 80.635) (end 208.65 80.635) (width 0.6) (layer "F.Cu") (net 2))
 (segment (start 202.827 82.805) (end 200.083 85.549) (width 0.6) (layer "F.Cu") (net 2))
 (segment (start 205 80) (end 205 81.272792) (width 0.6) (layer "F.Cu") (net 2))
 (segment (start 200.083 85.549) (end 197.611 85.549) (width 0.6) (layer "F.Cu") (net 2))
 (segment (start 205 81.272792) (end 203.467792 82.805) (width 0.6) (layer "F.Cu") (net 2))
 (segment (start 205 73.3) (end 205 80) (width 0.6) (layer "F.Cu") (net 2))
 (segment (start 199 68) (end 199.7 68) (width 0.6) (layer "F.Cu") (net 2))
 (segment (start 197.611 85.549) (end 196.16 87) (width 0.6) (layer "F.Cu") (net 2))
 (segment (start 201.35 80.635) (end 199.365 80.635) (width 0.6) (layer "F.Cu") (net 7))
 (segment (start 196 84) (end 196 84.62) (width 0.6) (layer "F.Cu") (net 7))
 (segment (start 199.365 80.635) (end 196 84) (width 0.6) (layer "F.Cu") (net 7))
 (segment (start 196 84.62) (end 193.62 87) (width 0.6) (layer "F.Cu") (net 7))
 (segment (start 208.65 81.905) (end 206.335 81.905) (width 0.6) (layer "F.Cu") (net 1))
 (segment (start 206.335 81.905) (end 201.24 87) (width 0.6) (layer "F.Cu") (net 1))
 (segment (start 207 60) (end 207 79.165) (width 0.6) (layer "F.Cu") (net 3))
 (segment (start 211 90) (end 201.7 90) (width 0.6) (layer "F.Cu") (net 3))
 (segment (start 208.65 79.365) (end 210.365 79.365) (width 0.6) (layer "F.Cu") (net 3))
 (segment (start 210.365 79.365) (end 211 80) (width 0.6) (layer "F.Cu") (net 3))
 (segment (start 201.7 90) (end 198.7 87) (width 0.6) (layer "F.Cu") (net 3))
 (segment (start 211 80) (end 211 90) (width 0.6) (layer "F.Cu") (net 3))
 (segment (start 207.2 79.365) (end 208.65 79.365) (width 0.6) (layer "F.Cu") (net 3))
 (segment (start 207 79.165) (end 207.2 79.365) (width 0.6) (layer "F.Cu") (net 3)))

